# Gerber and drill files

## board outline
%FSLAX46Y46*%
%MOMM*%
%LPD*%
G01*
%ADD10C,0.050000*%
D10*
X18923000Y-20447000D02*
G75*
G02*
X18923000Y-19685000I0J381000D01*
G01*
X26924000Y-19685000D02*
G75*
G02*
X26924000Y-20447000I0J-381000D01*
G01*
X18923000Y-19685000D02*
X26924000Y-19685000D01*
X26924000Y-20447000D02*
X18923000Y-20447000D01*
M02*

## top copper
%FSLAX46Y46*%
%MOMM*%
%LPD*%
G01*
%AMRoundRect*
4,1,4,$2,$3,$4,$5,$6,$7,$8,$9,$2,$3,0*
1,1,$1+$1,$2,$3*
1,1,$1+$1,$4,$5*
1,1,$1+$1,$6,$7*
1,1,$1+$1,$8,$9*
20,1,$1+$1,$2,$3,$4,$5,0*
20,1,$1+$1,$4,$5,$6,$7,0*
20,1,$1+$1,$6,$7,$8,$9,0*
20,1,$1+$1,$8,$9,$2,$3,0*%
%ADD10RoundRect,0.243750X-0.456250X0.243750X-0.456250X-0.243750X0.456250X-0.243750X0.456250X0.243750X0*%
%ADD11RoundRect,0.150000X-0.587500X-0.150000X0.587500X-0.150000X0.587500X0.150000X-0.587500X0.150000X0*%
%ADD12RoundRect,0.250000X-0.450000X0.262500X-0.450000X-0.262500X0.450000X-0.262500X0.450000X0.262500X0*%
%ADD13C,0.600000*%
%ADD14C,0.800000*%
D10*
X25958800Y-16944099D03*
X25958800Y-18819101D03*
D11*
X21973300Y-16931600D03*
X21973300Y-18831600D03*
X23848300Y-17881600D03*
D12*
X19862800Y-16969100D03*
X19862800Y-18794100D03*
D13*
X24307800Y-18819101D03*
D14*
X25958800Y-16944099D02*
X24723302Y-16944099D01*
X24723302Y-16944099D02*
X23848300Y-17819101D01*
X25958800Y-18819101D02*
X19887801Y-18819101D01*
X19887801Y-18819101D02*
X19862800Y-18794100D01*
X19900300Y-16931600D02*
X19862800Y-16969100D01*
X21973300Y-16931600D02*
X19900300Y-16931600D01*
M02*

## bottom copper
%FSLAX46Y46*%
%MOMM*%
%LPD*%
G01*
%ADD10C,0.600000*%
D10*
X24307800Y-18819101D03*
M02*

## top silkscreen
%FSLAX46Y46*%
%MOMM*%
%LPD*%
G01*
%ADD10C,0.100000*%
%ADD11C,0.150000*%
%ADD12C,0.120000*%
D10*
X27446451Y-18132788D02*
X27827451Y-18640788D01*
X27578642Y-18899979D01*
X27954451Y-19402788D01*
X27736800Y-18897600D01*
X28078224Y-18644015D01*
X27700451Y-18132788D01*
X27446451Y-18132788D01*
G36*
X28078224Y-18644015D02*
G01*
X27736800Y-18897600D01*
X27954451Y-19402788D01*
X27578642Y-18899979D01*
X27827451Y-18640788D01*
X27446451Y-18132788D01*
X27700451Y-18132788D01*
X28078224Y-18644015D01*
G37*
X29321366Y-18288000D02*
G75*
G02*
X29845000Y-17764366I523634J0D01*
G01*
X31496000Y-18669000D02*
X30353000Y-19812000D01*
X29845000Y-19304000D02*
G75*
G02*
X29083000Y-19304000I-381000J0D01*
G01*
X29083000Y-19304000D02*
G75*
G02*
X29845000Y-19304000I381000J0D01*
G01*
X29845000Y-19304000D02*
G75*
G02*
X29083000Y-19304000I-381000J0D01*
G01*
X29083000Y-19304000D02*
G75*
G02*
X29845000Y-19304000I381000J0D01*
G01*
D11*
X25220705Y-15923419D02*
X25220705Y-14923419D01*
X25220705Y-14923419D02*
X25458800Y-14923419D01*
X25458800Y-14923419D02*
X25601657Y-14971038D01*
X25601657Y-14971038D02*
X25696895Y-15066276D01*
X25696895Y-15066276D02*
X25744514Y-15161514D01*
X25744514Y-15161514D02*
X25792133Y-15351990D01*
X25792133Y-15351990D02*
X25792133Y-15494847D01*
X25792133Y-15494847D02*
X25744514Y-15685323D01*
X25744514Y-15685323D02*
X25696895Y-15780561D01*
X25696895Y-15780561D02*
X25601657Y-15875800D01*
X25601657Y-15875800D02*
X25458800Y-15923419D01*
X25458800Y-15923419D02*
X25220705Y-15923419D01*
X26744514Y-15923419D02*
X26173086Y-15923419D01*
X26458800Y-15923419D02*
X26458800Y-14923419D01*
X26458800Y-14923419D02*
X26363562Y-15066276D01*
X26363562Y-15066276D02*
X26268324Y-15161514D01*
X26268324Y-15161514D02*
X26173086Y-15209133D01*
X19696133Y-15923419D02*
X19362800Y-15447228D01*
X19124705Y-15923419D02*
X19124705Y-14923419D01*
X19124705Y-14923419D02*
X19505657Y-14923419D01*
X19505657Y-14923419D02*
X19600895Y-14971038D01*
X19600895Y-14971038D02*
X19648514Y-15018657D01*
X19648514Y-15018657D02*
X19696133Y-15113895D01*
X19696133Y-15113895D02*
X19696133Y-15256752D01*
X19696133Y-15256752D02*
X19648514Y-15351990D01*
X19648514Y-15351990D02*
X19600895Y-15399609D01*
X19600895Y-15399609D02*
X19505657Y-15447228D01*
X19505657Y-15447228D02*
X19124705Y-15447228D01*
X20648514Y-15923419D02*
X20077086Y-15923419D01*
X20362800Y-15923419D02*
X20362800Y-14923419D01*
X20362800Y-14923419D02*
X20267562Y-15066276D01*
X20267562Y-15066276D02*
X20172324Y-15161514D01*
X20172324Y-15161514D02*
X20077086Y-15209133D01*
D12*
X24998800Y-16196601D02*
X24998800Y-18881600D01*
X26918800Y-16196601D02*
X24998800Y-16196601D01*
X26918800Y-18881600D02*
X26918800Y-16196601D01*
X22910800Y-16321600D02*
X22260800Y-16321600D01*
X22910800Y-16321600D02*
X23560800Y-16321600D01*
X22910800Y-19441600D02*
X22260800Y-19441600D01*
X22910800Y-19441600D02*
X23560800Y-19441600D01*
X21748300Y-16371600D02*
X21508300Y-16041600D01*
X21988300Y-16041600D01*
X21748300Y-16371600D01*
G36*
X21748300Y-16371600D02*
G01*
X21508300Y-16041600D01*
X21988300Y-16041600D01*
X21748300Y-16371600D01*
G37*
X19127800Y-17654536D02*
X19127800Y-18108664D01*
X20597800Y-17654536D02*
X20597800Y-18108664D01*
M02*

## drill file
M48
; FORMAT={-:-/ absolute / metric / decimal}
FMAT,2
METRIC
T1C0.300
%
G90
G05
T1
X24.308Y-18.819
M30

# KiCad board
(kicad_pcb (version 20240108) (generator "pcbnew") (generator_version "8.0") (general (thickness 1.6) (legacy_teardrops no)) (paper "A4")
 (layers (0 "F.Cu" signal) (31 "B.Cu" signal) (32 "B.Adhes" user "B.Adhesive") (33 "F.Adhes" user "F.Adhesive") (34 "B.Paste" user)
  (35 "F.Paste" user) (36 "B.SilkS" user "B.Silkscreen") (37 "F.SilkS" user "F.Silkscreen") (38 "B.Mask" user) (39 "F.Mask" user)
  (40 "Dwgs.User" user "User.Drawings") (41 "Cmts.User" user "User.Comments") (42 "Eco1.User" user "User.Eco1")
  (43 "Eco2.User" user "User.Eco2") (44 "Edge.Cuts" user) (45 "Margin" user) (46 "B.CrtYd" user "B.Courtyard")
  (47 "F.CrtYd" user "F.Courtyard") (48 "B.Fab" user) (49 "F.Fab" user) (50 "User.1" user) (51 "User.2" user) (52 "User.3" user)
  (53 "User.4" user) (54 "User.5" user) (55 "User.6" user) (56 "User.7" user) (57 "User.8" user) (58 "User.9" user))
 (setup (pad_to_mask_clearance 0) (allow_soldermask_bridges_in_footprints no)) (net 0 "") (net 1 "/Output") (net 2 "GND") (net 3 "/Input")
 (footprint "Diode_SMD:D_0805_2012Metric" (layer "F.Cu") (at 25.9588 17.8816 -90)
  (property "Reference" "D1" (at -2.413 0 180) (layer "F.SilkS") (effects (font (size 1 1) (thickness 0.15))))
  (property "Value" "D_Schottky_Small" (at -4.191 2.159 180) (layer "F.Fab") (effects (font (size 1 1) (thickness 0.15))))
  (fp_line (start -1.684999 0.96) (end 1 0.96) (stroke (width 0.12) (type solid)) (layer "F.SilkS"))
  (fp_line (start -1.684999 -0.96) (end -1.684999 0.96) (stroke (width 0.12) (type solid)) (layer "F.SilkS"))
  (fp_line (start 1 -0.96) (end -1.684999 -0.96) (stroke (width 0.12) (type solid)) (layer "F.SilkS"))
  (pad "1" smd roundrect (at -0.937501 0 270) (size 0.975 1.4) (layers "F.Cu" "F.Paste" "F.Mask") (roundrect_rratio 0.25) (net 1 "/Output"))
  (pad "2" smd roundrect (at 0.937501 0 270) (size 0.975 1.4) (layers "F.Cu" "F.Paste" "F.Mask") (roundrect_rratio 0.25) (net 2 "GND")))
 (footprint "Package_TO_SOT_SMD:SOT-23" (layer "F.Cu") (at 22.9108 17.8816)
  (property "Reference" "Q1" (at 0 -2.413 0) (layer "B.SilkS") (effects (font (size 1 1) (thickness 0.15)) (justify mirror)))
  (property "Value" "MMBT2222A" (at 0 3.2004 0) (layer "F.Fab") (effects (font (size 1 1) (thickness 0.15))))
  (fp_line (start 0 -1.56) (end -0.65 -1.56) (stroke (width 0.12) (type solid)) (layer "F.SilkS"))
  (fp_line (start 0 -1.56) (end 0.65 -1.56) (stroke (width 0.12) (type solid)) (layer "F.SilkS"))
  (fp_line (start 0 1.56) (end -0.65 1.56) (stroke (width 0.12) (type solid)) (layer "F.SilkS"))
  (fp_line (start 0 1.56) (end 0.65 1.56) (stroke (width 0.12) (type solid)) (layer "F.SilkS"))
  (fp_poly
   (pts (xy -1.1625 -1.51) (xy -1.4025 -1.84) (xy -0.9225 -1.84) (xy -1.1625 -1.51)) (stroke (width 0.12) (type solid)) (fill solid)
   (layer "F.SilkS"))
  (pad "1" smd roundrect (at -0.9375 -0.95) (size 1.475 0.6) (layers "F.Cu" "F.Paste" "F.Mask") (roundrect_rratio 0.25) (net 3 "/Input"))
  (pad "2" smd roundrect (at -0.9375 0.95) (size 1.475 0.6) (layers "F.Cu" "F.Paste" "F.Mask") (roundrect_rratio 0.25) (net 2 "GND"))
  (pad "3" smd roundrect (at 0.9375 0) (size 1.475 0.6) (layers "F.Cu" "F.Paste" "F.Mask") (roundrect_rratio 0.25) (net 1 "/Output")))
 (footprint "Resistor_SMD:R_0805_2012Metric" (layer "F.Cu") (at 19.8628 17.8816 -90)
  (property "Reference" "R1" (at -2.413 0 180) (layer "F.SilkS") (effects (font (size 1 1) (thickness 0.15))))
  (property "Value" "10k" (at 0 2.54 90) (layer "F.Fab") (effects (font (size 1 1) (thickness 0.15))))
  (fp_line (start -0.227064 0.735) (end 0.227064 0.735) (stroke (width 0.12) (type solid)) (layer "F.SilkS"))
  (fp_line (start -0.227064 -0.735) (end 0.227064 -0.735) (stroke (width 0.12) (type solid)) (layer "F.SilkS"))
  (pad "1" smd roundrect (at -0.9125 0 270) (size 1.025 1.4) (layers "F.Cu" "F.Paste" "F.Mask") (roundrect_rratio 0.243902) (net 3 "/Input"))
  (pad "2" smd roundrect (at 0.9125 0 270) (size 1.025 1.4) (layers "F.Cu" "F.Paste" "F.Mask") (roundrect_rratio 0.243902) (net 2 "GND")))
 (gr_poly
  (pts (xy 27.446451 18.132788) (xy 27.827451 18.640788) (xy 27.578642 18.899979) (xy 27.954451 19.402788) (xy 27.7368 18.8976)
   (xy 28.078224 18.644015) (xy 27.700451 18.132788))
  (stroke (width 0.1) (type solid)) (fill solid) (layer "F.SilkS"))
 (gr_arc (start 29.321366 18.288) (mid 29.474735 17.917735) (end 29.845 17.764366) (stroke (width 0.1) (type default)) (layer "F.SilkS"))
 (gr_line (start 31.496 18.669) (end 30.353 19.812) (stroke (width 0.1) (type default)) (layer "F.SilkS"))
 (gr_circle (center 29.464 19.304) (end 29.464 18.923) (stroke (width 0.1) (type default)) (fill none) (layer "F.SilkS"))
 (gr_circle (center 29.464 19.304) (end 29.464 18.923) (stroke (width 0.1) (type default)) (fill none) (layer "F.SilkS"))
 (gr_arc (start 18.923 20.447) (mid 18.542 20.066) (end 18.923 19.685) (stroke (width 0.05) (type default)) (layer "Edge.Cuts"))
 (gr_arc (start 26.924 19.685) (mid 27.305 20.066) (end 26.924 20.447) (stroke (width 0.05) (type default)) (layer "Edge.Cuts"))
 (gr_line (start 18.923 19.685) (end 26.924 19.685) (stroke (width 0.05) (type default)) (layer "Edge.Cuts"))
 (gr_line (start 26.924 20.447) (end 18.923 20.447) (stroke (width 0.05) (type default)) (layer "Edge.Cuts"))
 (segment (start 25.9588 16.944099) (end 24.723302 16.944099) (width 0.8) (layer "F.Cu") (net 1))
 (segment (start 24.723302 16.944099) (end 23.8483 17.819101) (width 0.8) (layer "F.Cu") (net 1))
 (segment (start 25.9588 18.819101) (end 19.887801 18.819101) (width 0.8) (layer "F.Cu") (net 2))
 (segment (start 19.887801 18.819101) (end 19.8628 18.7941) (width 0.8) (layer "F.Cu") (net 2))
 (via (at 24.3078 18.819101) (size 0.6) (drill 0.3) (layers "F.Cu" "B.Cu") (free yes) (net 2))
 (segment (start 19.9003 16.9316) (end 19.8628 16.9691) (width 0.8) (layer "F.Cu") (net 3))
 (segment (start 21.9733 16.9316) (end 19.9003 16.9316) (width 0.8) (layer "F.Cu") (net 3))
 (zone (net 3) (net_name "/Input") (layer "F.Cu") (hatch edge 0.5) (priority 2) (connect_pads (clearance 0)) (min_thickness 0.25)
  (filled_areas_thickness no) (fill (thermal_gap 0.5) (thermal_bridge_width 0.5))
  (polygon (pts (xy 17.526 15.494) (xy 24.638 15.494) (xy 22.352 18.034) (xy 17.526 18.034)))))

